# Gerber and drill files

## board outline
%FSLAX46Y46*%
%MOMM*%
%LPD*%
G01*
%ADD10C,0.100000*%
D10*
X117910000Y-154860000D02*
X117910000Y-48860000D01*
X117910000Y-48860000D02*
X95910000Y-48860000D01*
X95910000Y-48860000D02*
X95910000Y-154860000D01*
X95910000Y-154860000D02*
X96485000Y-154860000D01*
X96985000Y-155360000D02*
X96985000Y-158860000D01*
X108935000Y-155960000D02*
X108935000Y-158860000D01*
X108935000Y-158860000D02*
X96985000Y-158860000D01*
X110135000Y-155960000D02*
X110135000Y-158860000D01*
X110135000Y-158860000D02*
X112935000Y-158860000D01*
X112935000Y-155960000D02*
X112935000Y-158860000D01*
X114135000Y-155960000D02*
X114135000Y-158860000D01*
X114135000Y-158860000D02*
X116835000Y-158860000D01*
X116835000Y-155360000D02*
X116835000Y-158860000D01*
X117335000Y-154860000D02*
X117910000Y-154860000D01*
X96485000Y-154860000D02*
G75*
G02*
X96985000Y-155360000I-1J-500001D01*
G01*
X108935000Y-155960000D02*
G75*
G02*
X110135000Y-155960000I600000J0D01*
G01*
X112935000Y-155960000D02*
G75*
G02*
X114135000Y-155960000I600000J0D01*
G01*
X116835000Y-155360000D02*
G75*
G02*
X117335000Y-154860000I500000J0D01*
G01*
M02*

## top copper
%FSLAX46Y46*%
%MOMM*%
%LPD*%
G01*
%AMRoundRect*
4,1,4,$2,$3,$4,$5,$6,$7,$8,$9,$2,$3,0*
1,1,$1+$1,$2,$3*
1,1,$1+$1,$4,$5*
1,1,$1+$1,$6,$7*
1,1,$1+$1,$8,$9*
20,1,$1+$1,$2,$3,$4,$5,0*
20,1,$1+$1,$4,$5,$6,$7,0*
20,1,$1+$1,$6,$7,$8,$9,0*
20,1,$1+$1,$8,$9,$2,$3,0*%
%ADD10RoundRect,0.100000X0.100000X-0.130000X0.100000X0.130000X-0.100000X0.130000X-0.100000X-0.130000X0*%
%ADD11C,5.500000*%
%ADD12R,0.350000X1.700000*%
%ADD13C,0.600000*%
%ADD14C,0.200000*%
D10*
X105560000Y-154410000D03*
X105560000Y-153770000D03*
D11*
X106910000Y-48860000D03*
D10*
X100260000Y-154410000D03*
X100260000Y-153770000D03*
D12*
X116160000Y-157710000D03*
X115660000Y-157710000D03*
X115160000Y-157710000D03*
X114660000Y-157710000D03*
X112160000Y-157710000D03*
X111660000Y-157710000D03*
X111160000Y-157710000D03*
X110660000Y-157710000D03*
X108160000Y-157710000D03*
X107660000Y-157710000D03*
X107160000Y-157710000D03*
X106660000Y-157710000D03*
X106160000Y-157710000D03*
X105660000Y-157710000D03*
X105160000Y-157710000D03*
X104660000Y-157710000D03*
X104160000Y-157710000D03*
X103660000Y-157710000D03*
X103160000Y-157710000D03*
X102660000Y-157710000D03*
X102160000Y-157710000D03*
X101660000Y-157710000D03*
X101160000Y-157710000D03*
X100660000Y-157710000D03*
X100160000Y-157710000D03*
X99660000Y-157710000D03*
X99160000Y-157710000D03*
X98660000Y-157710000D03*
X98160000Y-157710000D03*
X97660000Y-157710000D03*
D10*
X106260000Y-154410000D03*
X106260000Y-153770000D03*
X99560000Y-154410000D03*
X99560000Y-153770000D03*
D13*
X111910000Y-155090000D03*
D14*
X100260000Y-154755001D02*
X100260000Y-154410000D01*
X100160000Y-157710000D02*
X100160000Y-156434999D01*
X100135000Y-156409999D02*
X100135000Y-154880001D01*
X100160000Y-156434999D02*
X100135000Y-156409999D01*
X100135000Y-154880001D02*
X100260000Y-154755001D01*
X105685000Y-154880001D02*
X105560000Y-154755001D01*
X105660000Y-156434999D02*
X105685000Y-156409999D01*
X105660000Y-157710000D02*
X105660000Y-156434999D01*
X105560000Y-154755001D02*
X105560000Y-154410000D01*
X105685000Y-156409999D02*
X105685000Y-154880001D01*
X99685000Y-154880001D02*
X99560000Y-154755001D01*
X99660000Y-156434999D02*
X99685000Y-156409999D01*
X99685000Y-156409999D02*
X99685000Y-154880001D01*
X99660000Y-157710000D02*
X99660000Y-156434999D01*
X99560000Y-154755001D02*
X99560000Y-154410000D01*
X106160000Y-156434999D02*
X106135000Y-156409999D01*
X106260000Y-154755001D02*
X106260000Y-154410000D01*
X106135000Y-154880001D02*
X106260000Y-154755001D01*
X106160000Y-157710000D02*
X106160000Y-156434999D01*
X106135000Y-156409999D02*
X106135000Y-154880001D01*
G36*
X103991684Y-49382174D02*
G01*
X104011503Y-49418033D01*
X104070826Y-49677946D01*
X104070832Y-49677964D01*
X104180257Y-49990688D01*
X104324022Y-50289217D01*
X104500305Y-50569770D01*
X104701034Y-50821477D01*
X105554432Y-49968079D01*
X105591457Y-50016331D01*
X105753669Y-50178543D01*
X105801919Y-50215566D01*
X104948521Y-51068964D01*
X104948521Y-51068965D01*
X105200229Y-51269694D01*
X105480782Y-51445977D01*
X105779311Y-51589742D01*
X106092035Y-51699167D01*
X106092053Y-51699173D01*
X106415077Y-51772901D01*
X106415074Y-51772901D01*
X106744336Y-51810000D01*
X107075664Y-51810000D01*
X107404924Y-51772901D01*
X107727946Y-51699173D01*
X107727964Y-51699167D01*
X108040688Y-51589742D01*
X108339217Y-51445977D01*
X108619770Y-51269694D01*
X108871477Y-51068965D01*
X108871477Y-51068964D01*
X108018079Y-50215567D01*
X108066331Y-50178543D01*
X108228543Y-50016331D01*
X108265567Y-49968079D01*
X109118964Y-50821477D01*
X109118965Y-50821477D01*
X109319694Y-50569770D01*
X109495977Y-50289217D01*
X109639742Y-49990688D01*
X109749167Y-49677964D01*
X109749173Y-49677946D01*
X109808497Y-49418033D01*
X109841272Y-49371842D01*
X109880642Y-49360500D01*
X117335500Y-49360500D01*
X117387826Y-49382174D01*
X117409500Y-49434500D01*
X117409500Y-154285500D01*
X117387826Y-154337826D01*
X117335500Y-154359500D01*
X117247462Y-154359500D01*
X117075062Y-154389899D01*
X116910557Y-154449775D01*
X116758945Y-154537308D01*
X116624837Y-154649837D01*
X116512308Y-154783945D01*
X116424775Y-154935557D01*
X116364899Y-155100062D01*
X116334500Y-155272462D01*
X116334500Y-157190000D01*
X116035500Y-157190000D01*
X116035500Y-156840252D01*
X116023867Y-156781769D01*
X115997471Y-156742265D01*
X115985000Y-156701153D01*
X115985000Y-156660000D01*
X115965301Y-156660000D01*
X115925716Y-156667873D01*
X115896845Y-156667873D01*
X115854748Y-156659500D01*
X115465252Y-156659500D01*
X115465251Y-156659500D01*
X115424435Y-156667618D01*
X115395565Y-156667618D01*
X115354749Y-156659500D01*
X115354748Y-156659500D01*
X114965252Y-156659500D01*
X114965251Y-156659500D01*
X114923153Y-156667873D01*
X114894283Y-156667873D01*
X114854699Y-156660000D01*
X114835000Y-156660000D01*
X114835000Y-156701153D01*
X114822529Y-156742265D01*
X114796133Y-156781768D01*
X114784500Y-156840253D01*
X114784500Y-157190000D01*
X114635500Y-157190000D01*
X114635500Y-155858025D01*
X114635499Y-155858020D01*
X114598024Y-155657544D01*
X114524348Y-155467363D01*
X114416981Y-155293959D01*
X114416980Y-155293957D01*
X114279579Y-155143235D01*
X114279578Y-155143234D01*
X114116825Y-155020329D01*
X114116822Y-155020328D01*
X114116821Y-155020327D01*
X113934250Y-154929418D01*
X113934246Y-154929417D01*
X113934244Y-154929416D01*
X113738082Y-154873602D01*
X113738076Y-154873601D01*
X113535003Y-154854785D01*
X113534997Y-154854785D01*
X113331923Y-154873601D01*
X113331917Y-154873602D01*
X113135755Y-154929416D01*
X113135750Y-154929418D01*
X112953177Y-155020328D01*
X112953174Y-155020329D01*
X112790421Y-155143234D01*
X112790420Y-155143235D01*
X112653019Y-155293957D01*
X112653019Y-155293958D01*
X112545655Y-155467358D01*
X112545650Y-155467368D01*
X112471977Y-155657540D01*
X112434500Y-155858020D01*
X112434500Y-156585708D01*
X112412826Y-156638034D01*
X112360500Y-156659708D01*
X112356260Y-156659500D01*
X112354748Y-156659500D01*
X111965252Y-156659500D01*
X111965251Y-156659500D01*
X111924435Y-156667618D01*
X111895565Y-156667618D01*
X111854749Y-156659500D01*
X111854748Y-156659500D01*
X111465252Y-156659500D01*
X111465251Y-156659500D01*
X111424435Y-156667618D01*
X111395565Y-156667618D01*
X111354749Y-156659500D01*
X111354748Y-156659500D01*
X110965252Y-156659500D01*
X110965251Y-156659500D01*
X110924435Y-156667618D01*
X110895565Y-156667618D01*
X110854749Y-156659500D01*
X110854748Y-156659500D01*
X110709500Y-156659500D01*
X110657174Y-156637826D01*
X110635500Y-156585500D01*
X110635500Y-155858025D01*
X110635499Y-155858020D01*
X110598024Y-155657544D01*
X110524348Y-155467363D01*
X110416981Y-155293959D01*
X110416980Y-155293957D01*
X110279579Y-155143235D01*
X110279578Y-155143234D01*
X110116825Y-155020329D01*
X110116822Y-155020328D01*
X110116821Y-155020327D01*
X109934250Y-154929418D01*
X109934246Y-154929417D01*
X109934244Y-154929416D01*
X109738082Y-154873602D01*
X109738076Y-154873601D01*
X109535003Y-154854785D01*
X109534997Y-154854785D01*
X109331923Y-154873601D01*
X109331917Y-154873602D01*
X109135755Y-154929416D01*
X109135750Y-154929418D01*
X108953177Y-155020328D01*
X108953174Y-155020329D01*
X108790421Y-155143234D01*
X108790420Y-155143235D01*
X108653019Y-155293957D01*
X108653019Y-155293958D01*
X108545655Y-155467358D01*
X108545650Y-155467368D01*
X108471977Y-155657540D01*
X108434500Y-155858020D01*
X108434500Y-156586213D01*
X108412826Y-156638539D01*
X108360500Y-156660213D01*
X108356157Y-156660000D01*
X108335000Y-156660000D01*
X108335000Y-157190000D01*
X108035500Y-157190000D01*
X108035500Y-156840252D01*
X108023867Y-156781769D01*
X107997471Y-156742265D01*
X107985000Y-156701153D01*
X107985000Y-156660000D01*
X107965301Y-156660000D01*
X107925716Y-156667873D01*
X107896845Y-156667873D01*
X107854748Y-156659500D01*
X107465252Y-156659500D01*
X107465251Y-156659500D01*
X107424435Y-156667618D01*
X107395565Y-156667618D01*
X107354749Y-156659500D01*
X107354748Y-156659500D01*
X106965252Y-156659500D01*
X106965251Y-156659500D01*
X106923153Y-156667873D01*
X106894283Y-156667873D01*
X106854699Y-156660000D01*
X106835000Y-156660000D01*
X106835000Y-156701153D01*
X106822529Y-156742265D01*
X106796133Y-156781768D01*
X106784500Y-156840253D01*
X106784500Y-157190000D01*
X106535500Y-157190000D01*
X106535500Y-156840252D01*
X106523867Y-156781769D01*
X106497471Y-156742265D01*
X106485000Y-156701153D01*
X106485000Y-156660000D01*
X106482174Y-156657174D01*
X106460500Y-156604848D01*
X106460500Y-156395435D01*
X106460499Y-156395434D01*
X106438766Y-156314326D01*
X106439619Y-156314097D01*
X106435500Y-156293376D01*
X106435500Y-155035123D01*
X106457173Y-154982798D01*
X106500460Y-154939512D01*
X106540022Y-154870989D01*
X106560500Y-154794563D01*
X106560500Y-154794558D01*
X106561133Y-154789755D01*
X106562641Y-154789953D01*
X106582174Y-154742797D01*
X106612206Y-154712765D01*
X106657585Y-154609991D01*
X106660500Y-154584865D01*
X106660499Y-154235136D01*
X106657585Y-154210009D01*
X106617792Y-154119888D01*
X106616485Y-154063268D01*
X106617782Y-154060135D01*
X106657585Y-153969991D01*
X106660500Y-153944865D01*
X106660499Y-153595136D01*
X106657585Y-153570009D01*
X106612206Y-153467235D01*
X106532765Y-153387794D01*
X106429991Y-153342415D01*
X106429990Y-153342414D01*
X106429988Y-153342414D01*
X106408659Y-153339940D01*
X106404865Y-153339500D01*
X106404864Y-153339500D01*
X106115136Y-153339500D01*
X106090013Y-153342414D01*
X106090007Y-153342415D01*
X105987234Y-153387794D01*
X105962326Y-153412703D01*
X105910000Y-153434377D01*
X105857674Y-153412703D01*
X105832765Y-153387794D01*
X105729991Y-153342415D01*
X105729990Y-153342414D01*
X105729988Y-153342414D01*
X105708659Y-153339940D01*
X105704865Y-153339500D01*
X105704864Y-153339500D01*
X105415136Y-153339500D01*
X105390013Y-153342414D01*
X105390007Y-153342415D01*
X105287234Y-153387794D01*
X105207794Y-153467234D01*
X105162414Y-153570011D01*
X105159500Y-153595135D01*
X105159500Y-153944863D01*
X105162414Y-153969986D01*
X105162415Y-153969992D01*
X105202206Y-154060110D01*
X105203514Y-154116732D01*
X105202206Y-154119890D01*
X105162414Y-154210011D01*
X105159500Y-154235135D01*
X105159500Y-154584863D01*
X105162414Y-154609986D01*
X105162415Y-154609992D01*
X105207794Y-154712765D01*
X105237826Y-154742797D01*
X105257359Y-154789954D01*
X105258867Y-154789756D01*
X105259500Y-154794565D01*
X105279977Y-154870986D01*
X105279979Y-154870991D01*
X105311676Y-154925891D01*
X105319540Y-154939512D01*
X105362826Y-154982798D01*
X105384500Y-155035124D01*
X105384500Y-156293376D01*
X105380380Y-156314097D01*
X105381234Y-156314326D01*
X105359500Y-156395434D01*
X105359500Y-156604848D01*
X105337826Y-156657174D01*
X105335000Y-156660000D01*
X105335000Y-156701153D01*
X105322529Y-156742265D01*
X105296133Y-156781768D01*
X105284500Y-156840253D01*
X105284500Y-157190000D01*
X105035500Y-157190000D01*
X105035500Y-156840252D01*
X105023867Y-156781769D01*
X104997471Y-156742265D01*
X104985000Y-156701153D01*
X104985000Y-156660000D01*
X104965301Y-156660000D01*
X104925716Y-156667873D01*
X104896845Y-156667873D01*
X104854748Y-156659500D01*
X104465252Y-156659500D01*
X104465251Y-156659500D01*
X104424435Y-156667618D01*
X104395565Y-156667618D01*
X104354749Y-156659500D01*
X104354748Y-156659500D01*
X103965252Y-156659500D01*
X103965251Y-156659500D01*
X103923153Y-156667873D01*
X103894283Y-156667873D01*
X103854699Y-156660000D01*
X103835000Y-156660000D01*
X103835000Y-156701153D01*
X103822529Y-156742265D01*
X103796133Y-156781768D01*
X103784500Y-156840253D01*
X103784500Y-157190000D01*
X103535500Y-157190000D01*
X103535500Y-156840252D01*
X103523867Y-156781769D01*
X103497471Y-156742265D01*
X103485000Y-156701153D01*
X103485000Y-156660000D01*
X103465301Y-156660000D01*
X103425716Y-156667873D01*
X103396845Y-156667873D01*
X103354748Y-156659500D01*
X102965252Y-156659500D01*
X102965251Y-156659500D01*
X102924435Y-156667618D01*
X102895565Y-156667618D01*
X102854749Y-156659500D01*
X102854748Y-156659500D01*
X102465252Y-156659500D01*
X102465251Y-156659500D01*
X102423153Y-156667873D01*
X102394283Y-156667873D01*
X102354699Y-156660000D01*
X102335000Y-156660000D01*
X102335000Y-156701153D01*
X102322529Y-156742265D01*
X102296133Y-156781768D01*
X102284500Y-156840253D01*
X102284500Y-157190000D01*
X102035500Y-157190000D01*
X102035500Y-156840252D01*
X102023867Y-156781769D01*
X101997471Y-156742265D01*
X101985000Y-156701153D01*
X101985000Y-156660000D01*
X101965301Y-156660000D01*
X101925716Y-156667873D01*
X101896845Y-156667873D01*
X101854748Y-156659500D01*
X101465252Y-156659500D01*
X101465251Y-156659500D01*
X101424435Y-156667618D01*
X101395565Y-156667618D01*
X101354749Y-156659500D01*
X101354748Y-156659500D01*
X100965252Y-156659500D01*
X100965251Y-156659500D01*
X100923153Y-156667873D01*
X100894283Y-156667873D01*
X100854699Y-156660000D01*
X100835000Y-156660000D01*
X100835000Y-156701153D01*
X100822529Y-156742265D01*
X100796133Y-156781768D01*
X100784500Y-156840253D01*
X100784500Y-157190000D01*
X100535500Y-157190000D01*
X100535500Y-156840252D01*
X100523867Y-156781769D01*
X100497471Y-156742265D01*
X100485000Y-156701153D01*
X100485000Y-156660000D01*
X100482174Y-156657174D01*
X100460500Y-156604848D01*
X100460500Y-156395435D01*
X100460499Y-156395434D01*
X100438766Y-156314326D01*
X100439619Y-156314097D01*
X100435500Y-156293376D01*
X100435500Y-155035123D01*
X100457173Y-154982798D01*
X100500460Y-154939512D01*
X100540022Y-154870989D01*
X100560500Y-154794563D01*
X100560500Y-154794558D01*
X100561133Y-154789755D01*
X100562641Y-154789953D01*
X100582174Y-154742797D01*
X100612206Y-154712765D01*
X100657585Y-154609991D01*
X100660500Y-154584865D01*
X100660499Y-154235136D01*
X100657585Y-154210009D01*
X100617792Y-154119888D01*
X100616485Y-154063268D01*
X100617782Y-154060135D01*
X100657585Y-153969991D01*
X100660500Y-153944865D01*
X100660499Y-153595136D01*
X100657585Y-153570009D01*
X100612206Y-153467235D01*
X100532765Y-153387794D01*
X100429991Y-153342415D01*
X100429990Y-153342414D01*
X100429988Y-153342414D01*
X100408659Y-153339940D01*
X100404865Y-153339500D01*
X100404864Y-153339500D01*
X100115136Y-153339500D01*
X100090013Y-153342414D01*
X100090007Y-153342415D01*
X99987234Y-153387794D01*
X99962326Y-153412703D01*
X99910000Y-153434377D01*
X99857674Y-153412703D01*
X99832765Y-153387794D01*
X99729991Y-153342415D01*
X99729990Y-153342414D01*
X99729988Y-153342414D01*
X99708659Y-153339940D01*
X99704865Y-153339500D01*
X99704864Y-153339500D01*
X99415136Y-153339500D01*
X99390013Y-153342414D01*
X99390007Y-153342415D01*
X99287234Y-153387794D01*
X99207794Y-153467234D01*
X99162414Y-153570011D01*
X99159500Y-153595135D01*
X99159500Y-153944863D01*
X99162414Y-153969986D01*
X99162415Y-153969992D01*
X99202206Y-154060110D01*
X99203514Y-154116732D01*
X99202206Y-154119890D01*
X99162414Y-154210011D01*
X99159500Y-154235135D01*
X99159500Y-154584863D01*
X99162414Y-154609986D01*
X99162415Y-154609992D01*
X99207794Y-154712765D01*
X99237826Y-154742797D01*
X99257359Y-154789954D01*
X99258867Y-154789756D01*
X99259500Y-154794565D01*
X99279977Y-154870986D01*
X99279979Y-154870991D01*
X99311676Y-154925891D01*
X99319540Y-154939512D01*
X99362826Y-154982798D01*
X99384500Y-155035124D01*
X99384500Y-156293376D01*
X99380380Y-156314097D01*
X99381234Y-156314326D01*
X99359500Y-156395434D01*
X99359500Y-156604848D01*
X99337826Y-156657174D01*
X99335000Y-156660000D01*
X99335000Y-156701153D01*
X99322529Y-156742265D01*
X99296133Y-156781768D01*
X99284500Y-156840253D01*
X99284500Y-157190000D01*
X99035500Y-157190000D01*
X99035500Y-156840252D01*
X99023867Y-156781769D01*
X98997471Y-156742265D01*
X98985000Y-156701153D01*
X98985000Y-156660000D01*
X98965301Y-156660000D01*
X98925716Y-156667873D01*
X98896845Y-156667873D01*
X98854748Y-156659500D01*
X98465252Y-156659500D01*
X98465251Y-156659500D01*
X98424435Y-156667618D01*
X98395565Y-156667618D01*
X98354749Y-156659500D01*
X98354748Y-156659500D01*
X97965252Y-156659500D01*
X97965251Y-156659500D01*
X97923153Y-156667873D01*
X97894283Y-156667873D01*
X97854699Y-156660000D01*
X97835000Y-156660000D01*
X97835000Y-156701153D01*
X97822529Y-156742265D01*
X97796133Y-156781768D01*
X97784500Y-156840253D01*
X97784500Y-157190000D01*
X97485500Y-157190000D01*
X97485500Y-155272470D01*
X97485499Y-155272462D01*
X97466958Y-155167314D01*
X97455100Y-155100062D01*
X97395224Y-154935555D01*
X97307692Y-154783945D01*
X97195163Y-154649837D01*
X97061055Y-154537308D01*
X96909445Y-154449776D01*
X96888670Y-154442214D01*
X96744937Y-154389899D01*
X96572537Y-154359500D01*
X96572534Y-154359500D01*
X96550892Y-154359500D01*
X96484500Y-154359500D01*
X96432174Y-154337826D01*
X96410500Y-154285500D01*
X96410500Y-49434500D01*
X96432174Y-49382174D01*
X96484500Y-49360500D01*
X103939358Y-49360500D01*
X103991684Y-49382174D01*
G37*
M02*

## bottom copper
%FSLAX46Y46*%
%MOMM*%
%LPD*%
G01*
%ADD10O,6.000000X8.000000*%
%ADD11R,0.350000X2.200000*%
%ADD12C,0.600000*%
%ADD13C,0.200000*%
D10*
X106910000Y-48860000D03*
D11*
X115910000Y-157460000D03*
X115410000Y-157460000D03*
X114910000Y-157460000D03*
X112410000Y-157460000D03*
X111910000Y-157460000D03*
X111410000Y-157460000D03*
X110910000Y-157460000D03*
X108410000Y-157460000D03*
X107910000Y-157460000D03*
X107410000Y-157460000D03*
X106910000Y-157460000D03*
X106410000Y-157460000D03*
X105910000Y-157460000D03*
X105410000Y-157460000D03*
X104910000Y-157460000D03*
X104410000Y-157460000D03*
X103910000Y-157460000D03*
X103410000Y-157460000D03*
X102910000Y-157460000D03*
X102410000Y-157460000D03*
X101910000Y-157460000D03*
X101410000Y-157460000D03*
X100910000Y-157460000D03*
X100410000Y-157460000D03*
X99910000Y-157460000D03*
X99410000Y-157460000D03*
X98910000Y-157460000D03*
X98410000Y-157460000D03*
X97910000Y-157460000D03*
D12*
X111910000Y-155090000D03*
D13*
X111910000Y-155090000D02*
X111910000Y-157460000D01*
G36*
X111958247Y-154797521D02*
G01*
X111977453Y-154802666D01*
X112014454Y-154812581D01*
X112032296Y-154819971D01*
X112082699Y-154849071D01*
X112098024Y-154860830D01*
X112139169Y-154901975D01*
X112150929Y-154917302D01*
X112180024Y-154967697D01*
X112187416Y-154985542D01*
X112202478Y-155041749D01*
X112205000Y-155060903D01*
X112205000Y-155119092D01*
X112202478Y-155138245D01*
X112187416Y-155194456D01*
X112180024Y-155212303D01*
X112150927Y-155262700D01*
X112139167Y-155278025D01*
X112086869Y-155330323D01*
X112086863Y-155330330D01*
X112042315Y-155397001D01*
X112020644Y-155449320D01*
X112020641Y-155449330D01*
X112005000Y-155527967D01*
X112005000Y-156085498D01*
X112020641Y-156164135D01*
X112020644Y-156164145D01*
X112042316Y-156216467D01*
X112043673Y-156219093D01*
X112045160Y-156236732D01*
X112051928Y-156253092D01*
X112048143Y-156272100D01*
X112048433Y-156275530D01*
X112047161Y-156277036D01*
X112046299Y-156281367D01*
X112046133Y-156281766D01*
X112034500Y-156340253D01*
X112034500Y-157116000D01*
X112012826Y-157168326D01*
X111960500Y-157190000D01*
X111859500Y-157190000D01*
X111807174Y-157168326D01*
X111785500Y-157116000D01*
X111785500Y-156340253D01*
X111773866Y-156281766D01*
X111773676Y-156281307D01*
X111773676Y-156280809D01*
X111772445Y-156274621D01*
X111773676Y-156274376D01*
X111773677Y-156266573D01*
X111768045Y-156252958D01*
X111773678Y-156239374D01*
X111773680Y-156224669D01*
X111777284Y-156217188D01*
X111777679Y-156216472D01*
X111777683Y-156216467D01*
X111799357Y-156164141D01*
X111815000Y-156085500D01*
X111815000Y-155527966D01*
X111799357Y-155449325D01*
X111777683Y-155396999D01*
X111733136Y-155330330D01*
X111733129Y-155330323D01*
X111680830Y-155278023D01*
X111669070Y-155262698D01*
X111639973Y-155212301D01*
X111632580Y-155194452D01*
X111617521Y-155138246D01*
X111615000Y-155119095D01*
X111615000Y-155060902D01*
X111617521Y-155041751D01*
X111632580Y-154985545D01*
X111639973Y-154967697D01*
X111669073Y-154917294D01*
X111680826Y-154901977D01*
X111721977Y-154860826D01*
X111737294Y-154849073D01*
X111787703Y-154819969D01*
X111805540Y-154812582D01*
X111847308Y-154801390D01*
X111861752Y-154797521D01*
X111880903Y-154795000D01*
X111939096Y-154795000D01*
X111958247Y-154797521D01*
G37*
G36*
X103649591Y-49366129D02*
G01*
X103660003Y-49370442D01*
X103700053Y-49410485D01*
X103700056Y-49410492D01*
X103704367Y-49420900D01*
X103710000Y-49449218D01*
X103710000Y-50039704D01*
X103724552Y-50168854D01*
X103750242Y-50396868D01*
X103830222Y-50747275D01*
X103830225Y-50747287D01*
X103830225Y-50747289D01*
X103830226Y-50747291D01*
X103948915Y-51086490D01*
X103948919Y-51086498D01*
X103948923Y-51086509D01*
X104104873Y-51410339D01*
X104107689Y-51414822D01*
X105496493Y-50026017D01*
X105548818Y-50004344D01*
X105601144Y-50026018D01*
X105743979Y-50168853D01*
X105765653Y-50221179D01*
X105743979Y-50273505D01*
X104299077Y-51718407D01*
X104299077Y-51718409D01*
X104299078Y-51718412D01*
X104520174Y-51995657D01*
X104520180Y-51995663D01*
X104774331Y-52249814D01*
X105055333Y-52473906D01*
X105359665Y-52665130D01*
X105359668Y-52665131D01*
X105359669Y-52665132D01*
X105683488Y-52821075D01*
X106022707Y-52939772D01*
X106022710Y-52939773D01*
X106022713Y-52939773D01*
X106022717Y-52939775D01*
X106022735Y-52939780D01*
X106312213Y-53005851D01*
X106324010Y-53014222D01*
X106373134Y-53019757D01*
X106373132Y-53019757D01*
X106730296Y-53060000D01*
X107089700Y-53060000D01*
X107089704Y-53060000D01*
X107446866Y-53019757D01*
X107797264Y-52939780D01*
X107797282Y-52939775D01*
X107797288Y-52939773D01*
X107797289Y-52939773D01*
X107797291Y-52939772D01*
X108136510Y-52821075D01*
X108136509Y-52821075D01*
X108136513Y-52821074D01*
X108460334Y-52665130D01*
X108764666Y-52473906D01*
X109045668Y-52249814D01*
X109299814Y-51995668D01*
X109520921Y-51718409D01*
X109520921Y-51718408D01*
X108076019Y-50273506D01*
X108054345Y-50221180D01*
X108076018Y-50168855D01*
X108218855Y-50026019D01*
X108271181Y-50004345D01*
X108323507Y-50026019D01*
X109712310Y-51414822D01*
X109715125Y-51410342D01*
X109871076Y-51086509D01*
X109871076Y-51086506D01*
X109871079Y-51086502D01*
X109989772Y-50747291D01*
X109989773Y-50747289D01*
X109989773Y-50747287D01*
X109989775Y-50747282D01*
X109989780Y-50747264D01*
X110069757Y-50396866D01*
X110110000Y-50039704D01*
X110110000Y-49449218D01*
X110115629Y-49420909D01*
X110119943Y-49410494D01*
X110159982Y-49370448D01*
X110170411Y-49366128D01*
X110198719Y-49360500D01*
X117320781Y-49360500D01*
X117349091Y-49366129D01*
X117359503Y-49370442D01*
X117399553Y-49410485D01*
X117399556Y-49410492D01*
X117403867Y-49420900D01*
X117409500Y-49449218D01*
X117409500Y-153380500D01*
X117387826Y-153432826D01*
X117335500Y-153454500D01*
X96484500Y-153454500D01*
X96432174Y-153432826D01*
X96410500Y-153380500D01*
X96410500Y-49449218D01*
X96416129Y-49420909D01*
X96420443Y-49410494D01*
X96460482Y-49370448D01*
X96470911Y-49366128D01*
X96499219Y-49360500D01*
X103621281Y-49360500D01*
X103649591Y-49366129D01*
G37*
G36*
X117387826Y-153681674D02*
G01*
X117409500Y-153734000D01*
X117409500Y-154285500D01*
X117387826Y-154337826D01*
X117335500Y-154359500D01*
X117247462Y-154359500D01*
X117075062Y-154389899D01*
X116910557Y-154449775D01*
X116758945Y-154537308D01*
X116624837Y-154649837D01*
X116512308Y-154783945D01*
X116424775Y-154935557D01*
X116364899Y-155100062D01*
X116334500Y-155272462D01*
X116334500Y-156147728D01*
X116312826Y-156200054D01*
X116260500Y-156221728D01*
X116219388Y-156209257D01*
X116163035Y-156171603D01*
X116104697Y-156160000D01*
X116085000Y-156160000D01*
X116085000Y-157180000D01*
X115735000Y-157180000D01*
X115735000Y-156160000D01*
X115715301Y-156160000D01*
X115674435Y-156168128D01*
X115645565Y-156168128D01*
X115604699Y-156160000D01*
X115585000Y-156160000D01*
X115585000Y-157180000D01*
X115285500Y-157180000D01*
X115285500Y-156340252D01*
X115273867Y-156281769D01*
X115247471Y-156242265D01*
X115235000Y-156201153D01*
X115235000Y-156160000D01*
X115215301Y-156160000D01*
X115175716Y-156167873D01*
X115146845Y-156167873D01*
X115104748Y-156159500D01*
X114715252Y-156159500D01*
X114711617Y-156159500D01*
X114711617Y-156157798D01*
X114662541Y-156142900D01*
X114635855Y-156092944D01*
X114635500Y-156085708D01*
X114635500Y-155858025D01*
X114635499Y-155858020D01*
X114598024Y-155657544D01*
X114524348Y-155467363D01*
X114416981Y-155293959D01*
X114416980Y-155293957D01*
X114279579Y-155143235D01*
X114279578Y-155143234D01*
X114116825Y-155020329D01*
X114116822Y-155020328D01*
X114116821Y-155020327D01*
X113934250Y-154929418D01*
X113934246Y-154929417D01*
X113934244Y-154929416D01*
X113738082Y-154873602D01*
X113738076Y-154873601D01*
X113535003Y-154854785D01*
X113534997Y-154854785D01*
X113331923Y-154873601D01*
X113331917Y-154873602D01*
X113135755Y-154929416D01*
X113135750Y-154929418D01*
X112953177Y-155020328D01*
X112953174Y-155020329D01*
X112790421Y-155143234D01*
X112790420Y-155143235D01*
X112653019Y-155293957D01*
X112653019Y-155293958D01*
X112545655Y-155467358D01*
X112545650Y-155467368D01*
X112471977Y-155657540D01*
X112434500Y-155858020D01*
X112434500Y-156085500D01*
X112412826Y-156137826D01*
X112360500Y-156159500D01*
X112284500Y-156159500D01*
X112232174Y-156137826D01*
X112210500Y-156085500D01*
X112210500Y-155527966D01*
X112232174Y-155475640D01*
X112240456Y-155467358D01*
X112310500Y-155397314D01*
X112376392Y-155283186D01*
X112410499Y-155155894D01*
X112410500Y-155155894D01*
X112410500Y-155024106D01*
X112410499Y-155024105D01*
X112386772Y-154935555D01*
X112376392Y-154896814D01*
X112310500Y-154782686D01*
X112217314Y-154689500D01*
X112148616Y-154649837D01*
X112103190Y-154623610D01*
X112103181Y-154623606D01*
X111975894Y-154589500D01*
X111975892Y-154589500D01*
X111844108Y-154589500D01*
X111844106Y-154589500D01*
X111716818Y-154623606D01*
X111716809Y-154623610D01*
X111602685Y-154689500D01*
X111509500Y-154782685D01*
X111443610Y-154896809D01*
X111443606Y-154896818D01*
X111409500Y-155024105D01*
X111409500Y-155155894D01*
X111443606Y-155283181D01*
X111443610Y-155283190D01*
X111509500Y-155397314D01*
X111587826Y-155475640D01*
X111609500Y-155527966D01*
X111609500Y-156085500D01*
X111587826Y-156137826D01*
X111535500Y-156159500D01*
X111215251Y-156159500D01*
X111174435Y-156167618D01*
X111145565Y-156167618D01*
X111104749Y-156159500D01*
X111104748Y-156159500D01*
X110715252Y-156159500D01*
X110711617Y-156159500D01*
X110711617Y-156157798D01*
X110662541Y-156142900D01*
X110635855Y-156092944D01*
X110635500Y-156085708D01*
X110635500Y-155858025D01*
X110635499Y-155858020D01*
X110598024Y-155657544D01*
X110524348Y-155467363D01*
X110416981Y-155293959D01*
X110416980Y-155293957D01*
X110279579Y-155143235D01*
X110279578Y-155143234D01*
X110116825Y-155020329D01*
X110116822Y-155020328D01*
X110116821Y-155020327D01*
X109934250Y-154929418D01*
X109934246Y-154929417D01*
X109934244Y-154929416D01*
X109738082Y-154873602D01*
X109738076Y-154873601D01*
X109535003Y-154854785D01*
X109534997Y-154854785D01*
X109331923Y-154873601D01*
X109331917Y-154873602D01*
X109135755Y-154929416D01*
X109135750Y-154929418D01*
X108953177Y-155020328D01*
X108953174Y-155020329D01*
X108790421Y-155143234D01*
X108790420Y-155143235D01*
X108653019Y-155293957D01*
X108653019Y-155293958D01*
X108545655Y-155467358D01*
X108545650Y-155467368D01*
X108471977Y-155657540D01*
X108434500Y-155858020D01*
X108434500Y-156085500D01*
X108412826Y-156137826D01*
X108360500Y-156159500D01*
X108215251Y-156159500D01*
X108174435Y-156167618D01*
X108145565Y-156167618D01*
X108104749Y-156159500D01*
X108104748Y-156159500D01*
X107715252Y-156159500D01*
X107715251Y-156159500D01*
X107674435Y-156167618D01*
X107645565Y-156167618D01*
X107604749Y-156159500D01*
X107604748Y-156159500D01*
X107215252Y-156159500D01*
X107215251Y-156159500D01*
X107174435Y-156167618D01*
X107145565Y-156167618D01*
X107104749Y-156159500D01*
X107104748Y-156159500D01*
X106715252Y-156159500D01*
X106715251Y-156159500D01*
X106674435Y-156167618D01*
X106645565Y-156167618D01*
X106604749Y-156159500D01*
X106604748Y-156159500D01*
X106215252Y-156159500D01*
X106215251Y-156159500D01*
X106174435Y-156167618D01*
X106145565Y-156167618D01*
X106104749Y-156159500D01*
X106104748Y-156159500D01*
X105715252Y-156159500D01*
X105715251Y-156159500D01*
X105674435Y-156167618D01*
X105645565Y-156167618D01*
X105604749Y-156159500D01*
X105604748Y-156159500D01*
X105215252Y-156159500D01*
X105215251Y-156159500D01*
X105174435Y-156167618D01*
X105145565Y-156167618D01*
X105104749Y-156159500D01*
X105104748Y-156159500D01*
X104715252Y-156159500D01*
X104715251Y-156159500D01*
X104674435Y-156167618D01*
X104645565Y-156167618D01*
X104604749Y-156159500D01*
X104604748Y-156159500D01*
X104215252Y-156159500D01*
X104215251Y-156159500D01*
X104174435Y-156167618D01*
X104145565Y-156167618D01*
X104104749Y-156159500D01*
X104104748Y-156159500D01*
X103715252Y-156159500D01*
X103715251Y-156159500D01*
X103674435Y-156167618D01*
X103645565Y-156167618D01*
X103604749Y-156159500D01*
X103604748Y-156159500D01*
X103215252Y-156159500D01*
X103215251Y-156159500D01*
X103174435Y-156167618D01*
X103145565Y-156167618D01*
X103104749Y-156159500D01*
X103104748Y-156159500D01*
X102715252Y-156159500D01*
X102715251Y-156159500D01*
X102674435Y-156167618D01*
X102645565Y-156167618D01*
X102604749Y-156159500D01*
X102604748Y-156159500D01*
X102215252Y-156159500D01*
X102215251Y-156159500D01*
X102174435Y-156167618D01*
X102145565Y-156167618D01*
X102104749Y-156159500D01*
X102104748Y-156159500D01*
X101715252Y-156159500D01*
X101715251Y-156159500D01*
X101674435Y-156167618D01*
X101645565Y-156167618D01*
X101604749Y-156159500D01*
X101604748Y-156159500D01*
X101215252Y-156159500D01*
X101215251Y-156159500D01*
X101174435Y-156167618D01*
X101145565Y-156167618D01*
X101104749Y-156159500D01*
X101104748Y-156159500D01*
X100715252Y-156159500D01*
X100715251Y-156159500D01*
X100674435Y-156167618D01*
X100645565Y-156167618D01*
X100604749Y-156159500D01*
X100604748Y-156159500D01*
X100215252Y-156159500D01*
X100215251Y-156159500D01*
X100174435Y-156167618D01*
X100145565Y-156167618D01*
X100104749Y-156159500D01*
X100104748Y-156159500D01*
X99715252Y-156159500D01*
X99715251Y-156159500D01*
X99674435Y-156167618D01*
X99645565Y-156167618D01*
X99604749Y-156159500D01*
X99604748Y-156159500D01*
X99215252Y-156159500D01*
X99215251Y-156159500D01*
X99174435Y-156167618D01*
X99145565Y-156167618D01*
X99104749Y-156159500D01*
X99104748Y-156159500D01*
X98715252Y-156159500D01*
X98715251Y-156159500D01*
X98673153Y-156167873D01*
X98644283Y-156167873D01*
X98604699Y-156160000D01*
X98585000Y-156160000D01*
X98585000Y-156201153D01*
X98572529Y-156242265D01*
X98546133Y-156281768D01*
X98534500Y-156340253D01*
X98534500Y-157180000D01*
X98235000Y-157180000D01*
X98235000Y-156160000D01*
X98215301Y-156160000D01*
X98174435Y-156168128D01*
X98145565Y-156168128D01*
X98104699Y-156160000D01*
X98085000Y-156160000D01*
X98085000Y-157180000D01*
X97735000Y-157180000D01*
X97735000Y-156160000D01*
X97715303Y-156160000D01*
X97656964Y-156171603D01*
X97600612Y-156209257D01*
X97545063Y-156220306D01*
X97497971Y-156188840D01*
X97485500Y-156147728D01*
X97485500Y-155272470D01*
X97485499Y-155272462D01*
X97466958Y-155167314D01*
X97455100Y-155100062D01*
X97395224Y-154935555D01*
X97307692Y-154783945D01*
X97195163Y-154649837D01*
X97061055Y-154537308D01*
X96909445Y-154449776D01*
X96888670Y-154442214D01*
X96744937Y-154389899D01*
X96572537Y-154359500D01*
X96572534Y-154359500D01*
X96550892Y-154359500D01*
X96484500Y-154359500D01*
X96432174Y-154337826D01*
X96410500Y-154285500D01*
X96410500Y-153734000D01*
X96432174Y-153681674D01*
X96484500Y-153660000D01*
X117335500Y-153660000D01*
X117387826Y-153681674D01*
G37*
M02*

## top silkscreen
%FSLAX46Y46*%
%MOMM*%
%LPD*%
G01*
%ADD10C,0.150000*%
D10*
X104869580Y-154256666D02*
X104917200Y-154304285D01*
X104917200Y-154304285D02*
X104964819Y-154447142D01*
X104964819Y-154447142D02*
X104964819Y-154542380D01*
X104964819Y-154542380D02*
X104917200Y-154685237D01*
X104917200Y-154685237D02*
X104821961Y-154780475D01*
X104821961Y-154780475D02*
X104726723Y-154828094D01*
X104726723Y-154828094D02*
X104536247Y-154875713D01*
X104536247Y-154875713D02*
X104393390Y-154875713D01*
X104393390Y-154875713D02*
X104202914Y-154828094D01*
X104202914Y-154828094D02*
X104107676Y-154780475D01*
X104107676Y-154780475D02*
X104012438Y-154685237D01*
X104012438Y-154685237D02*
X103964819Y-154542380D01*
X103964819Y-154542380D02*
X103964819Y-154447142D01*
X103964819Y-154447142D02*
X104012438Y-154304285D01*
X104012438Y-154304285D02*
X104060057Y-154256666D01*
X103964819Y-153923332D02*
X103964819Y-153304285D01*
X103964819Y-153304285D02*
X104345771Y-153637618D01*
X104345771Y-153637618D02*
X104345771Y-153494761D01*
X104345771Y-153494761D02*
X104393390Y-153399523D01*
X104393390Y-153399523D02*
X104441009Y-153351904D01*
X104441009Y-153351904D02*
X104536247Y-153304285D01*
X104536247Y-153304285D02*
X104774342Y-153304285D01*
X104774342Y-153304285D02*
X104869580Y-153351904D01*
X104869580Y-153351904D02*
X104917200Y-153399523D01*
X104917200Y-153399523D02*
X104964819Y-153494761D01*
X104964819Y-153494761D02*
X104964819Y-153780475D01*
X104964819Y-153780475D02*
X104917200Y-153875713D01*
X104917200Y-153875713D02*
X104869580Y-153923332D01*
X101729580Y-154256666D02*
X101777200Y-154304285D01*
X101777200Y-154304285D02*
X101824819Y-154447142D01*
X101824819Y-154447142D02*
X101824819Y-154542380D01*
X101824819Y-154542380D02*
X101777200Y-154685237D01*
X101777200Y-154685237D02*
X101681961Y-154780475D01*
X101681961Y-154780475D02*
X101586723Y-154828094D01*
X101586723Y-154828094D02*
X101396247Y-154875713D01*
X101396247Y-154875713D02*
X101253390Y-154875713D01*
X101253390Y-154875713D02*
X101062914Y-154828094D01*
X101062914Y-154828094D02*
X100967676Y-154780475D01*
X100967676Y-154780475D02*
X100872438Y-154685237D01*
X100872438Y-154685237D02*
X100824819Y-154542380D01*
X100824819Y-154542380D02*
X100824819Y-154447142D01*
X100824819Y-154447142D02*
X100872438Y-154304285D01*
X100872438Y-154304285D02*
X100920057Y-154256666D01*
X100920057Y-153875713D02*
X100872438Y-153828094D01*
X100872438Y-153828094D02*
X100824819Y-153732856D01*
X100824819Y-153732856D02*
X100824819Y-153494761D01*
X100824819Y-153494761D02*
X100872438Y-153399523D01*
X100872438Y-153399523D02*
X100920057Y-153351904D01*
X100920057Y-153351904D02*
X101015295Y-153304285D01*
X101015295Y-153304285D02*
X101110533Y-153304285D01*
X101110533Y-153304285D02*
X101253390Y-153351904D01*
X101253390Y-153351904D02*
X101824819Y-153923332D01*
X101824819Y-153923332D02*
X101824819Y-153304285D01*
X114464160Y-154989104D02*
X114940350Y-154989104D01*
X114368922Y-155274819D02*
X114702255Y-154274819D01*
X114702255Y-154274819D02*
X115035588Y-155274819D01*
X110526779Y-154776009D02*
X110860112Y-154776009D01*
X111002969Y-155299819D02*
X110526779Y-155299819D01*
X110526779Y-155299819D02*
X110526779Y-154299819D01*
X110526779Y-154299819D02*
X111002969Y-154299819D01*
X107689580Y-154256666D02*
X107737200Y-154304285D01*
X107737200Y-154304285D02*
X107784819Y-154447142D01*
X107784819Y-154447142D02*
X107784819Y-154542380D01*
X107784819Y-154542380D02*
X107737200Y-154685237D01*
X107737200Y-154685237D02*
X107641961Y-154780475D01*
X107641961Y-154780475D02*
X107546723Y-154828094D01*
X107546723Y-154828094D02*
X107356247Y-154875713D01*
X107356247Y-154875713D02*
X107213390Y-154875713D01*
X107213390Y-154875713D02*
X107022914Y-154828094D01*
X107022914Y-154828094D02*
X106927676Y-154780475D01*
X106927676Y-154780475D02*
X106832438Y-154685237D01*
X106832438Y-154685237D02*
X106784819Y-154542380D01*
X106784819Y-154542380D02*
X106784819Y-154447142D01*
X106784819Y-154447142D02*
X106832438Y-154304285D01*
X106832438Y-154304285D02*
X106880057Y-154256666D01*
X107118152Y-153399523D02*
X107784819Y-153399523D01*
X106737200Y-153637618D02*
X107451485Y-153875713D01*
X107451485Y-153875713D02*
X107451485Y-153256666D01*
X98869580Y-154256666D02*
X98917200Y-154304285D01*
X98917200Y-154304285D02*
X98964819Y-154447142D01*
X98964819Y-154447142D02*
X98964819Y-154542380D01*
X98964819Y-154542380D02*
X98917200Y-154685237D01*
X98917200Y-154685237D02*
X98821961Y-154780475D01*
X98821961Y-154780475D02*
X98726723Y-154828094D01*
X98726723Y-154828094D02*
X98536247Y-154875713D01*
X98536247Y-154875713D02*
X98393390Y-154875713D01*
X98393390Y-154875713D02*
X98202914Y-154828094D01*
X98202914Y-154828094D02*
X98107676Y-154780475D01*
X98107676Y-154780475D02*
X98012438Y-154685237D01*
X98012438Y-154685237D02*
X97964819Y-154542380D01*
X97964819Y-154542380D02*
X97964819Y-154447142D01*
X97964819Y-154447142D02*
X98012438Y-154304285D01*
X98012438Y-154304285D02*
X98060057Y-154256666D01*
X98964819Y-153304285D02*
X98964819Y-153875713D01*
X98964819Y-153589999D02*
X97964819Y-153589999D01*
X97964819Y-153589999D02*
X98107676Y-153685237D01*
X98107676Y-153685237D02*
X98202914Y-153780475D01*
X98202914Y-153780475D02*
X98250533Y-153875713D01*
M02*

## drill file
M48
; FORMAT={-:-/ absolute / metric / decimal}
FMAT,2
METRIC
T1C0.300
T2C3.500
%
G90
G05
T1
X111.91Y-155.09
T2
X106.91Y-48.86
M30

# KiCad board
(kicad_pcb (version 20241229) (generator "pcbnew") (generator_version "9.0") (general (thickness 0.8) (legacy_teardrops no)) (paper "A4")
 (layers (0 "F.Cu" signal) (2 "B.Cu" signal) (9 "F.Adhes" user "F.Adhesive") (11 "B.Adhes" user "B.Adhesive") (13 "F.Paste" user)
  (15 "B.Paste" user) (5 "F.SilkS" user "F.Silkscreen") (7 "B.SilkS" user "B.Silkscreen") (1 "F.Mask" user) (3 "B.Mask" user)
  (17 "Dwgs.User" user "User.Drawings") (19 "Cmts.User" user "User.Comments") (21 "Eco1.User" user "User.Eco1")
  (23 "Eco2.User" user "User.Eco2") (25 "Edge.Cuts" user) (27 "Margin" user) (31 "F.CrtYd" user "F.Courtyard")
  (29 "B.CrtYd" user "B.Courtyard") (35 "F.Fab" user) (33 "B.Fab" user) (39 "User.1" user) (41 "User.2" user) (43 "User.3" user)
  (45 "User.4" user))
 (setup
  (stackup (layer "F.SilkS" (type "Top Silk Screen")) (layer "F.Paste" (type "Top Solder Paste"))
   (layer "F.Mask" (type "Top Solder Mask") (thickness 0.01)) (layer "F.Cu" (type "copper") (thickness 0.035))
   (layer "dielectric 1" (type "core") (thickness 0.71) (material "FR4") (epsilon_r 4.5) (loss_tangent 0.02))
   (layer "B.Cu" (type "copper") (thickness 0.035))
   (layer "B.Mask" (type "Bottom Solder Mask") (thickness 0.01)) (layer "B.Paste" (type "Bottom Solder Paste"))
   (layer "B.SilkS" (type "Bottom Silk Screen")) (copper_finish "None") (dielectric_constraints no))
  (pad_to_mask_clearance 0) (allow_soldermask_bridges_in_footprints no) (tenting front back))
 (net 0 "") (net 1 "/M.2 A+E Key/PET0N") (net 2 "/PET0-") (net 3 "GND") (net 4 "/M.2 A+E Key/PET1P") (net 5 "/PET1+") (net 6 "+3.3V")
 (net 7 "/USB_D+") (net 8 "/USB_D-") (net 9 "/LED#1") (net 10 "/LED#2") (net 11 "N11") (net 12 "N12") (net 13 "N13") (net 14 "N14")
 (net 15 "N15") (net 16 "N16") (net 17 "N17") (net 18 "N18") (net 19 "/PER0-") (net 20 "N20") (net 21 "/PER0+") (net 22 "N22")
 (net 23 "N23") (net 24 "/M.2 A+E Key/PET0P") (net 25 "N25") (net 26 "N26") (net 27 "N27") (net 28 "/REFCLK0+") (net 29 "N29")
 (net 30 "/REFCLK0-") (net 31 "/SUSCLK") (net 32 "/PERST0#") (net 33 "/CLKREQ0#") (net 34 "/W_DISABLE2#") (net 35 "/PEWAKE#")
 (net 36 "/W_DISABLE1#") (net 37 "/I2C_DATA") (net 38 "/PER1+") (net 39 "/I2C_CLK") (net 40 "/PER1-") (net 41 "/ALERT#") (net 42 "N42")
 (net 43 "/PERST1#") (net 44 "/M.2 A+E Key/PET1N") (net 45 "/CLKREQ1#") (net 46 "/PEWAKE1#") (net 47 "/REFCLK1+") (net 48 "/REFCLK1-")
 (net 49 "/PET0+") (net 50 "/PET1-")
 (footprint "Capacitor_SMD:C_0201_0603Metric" (layer "F.Cu") (at 105.56 154.09 90)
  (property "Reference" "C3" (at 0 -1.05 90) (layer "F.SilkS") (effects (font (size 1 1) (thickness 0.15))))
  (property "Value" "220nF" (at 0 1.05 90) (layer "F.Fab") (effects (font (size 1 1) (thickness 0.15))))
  (pad "" smd roundrect (at -0.345 0 90) (size 0.318 0.36) (layers "F.Paste") (roundrect_rratio 0.25))
  (pad "" smd roundrect (at 0.345 0 90) (size 0.318 0.36) (layers "F.Paste") (roundrect_rratio 0.25))
  (pad "1" smd roundrect (at -0.32 0 90) (size 0.46 0.4) (layers "F.Cu" "F.Mask") (roundrect_rratio 0.25) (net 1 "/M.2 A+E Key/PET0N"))
  (pad "2" smd roundrect (at 0.32 0 90) (size 0.46 0.4) (layers "F.Cu" "F.Mask") (roundrect_rratio 0.25) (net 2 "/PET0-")))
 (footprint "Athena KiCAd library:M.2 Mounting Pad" (layer "F.Cu") (at 106.91 48.86)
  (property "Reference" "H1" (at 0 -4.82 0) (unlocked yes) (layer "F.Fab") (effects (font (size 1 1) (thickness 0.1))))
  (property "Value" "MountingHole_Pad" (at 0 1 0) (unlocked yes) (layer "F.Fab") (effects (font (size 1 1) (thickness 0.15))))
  (pad "1" thru_hole circle (at 0 0) (size 5.5 5.5) (drill 3.5) (layers "*.Cu" "*.Mask") (remove_unused_layers no) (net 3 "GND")
   (padstack (mode front_inner_back)
    (layer "Inner" (shape circle) (size 5.5 5.5) (zone_connect -1))
    (layer "B.Cu" (shape oval) (size 6 8) (thermal_bridge_angle 45) (zone_connect -1)))))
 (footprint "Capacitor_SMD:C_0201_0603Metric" (layer "F.Cu") (at 100.26 154.09 90)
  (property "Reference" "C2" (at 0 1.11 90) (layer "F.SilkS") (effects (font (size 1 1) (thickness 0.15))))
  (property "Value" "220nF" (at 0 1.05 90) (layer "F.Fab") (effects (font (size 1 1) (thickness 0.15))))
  (pad "" smd roundrect (at -0.345 0 90) (size 0.318 0.36) (layers "F.Paste") (roundrect_rratio 0.25))
  (pad "" smd roundrect (at 0.345 0 90) (size 0.318 0.36) (layers "F.Paste") (roundrect_rratio 0.25))
  (pad "1" smd roundrect (at -0.32 0 90) (size 0.46 0.4) (layers "F.Cu" "F.Mask") (roundrect_rratio 0.25) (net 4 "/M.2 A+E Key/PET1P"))
  (pad "2" smd roundrect (at 0.32 0 90) (size 0.46 0.4) (layers "F.Cu" "F.Mask") (roundrect_rratio 0.25) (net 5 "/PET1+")))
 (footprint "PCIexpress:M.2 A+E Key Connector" (layer "F.Cu") (at 106.91 157.75)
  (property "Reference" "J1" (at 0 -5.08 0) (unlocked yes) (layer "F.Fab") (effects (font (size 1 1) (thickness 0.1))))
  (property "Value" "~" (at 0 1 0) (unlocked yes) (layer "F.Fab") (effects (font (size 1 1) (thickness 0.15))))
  (fp_line (start -11 -2.89) (end -10.425 -2.89) (stroke (width 0.1) (type default)) (layer "Edge.Cuts"))
  (fp_line (start -9.925 -2.39) (end -9.925 1.11) (stroke (width 0.1) (type default)) (layer "Edge.Cuts"))
  (fp_line (start 2.025 -1.79) (end 2.025 1.11) (stroke (width 0.1) (type default)) (layer "Edge.Cuts"))
  (fp_line (start 2.025 1.11) (end -9.925 1.11) (stroke (width 0.1) (type default)) (layer "Edge.Cuts"))
  (fp_line (start 3.225 -1.79) (end 3.225 1.11) (stroke (width 0.1) (type default)) (layer "Edge.Cuts"))
  (fp_line (start 3.225 1.11) (end 6.025 1.11) (stroke (width 0.1) (type default)) (layer "Edge.Cuts"))
  (fp_line (start 6.025 -1.79) (end 6.025 1.11) (stroke (width 0.1) (type default)) (layer "Edge.Cuts"))
  (fp_line (start 7.225 -1.79) (end 7.225 1.11) (stroke (width 0.1) (type default)) (layer "Edge.Cuts"))
  (fp_line (start 7.225 1.11) (end 9.925 1.11) (stroke (width 0.1) (type default)) (layer "Edge.Cuts"))
  (fp_line (start 9.925 -2.39) (end 9.925 1.11) (stroke (width 0.1) (type default)) (layer "Edge.Cuts"))
  (fp_line (start 10.425 -2.89) (end 11 -2.89) (stroke (width 0.1) (type default)) (layer "Edge.Cuts"))
  (fp_arc (start -10.425 -2.89) (mid -10.071447 -2.743553) (end -9.925 -2.39) (stroke (width 0.1) (type default)) (layer "Edge.Cuts"))
  (fp_arc (start 2.025 -1.79) (mid 2.625 -2.39) (end 3.225 -1.79) (stroke (width 0.1) (type default)) (layer "Edge.Cuts"))
  (fp_arc (start 6.025 -1.79) (mid 6.625 -2.39) (end 7.225 -1.79) (stroke (width 0.1) (type default)) (layer "Edge.Cuts"))
  (fp_arc (start 9.925 -2.39) (mid 10.071447 -2.743553) (end 10.425 -2.89) (stroke (width 0.1) (type default)) (layer "Edge.Cuts"))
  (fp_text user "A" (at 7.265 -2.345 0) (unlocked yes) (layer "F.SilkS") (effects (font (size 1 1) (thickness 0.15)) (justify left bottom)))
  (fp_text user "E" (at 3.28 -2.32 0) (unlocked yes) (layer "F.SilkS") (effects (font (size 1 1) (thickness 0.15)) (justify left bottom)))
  (pad "1" smd rect (at 9.25 -0.04 180) (size 0.35 1.7) (layers "F.Cu") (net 3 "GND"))
  (pad "2" smd rect (at 9 -0.29 180) (size 0.35 2.2) (layers "B.Cu") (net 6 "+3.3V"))
  (pad "3" smd rect (at 8.75 -0.04 180) (size 0.35 1.7) (layers "F.Cu") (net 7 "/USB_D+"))
  (pad "4" smd rect (at 8.5 -0.29 180) (size 0.35 2.2) (layers "B.Cu") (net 6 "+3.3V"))
  (pad "5" smd rect (at 8.25 -0.04 180) (size 0.35 1.7) (layers "F.Cu") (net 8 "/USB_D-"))
  (pad "6" smd rect (at 8 -0.29 180) (size 0.35 2.2) (layers "B.Cu") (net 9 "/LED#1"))
  (pad "7" smd rect (at 7.75 -0.04 180) (size 0.35 1.7) (layers "F.Cu") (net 3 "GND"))
  (pad "16" smd rect (at 5.5 -0.29 180) (size 0.35 2.2) (layers "B.Cu") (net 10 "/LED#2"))
  (pad "17" smd rect (at 5.25 -0.04 180) (size 0.35 1.7) (layers "F.Cu") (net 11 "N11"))
  (pad "18" smd rect (at 5 -0.29 180) (size 0.35 2.2) (layers "B.Cu") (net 3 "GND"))
  (pad "19" smd rect (at 4.75 -0.04 180) (size 0.35 1.7) (layers "F.Cu") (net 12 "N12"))
  (pad "20" smd rect (at 4.5 -0.29 180) (size 0.35 2.2) (layers "B.Cu") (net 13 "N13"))
  (pad "21" smd rect (at 4.25 -0.04 180) (size 0.35 1.7) (layers "F.Cu") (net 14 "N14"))
  (pad "22" smd rect (at 4 -0.29 180) (size 0.35 2.2) (layers "B.Cu") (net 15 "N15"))
  (pad "23" smd rect (at 3.75 -0.04 180) (size 0.35 1.7) (layers "F.Cu") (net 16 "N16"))
  (pad "32" smd rect (at 1.5 -0.29 180) (size 0.35 2.2) (layers "B.Cu") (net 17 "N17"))
  (pad "33" smd rect (at 1.25 -0.04 180) (size 0.35 1.7) (layers "F.Cu") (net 3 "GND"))
  (pad "34" smd rect (at 1 -0.29 180) (size 0.35 2.2) (layers "B.Cu") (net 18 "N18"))
  (pad "35" smd rect (at 0.75 -0.04 180) (size 0.35 1.7) (layers "F.Cu") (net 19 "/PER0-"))
  (pad "36" smd rect (at 0.5 -0.29 180) (size 0.35 2.2) (layers "B.Cu") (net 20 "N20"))
  (pad "37" smd rect (at 0.25 -0.04 180) (size 0.35 1.7) (layers "F.Cu") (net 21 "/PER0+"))
  (pad "38" smd rect (at 0 -0.29 180) (size 0.35 2.2) (layers "B.Cu") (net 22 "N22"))
  (pad "39" smd rect (at -0.25 -0.04 180) (size 0.35 1.7) (layers "F.Cu") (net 3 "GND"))
  (pad "40" smd rect (at -0.5 -0.29 180) (size 0.35 2.2) (layers "B.Cu") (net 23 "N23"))
  (pad "41" smd rect (at -0.75 -0.04 180) (size 0.35 1.7) (layers "F.Cu") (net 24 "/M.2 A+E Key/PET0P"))
  (pad "42" smd rect (at -1 -0.29 180) (size 0.35 2.2) (layers "B.Cu") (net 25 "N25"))
  (pad "43" smd rect (at -1.25 -0.04 180) (size 0.35 1.7) (layers "F.Cu") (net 1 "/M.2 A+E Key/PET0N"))
  (pad "44" smd rect (at -1.5 -0.29 180) (size 0.35 2.2) (layers "B.Cu") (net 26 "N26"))
  (pad "45" smd rect (at -1.75 -0.04 180) (size 0.35 1.7) (layers "F.Cu") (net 3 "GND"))
  (pad "46" smd rect (at -2 -0.29 180) (size 0.35 2.2) (layers "B.Cu") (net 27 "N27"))
  (pad "47" smd rect (at -2.25 -0.04 180) (size 0.35 1.7) (layers "F.Cu") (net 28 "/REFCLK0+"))
  (pad "48" smd rect (at -2.5 -0.29 180) (size 0.35 2.2) (layers "B.Cu") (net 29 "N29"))
  (pad "49" smd rect (at -2.75 -0.04 180) (size 0.35 1.7) (layers "F.Cu") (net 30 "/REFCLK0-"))
  (pad "50" smd rect (at -3 -0.29 180) (size 0.35 2.2) (layers "B.Cu") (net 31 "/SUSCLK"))
  (pad "51" smd rect (at -3.25 -0.04 180) (size 0.35 1.7) (layers "F.Cu") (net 3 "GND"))
  (pad "52" smd rect (at -3.5 -0.29 180) (size 0.35 2.2) (layers "B.Cu") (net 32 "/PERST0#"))
  (pad "53" smd rect (at -3.75 -0.04 180) (size 0.35 1.7) (layers "F.Cu") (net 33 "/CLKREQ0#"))
  (pad "54" smd rect (at -4 -0.29 180) (size 0.35 2.2) (layers "B.Cu") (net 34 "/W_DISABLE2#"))
  (pad "55" smd rect (at -4.25 -0.04 180) (size 0.35 1.7) (layers "F.Cu") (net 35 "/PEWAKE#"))
  (pad "56" smd rect (at -4.5 -0.29 180) (size 0.35 2.2) (layers "B.Cu") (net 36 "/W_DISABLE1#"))
  (pad "57" smd rect (at -4.75 -0.04 180) (size 0.35 1.7) (layers "F.Cu") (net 3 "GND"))
  (pad "58" smd rect (at -5 -0.29 180) (size 0.35 2.2) (layers "B.Cu") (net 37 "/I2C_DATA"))
  (pad "59" smd rect (at -5.25 -0.04 180) (size 0.35 1.7) (layers "F.Cu") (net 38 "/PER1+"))
  (pad "60" smd rect (at -5.5 -0.29 180) (size 0.35 2.2) (layers "B.Cu") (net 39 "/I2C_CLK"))
  (pad "61" smd rect (at -5.75 -0.04 180) (size 0.35 1.7) (layers "F.Cu") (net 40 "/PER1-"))
  (pad "62" smd rect (at -6 -0.29 180) (size 0.35 2.2) (layers "B.Cu") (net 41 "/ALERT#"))
  (pad "63" smd rect (at -6.25 -0.04 180) (size 0.35 1.7) (layers "F.Cu") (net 3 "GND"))
  (pad "64" smd rect (at -6.5 -0.29 180) (size 0.35 2.2) (layers "B.Cu") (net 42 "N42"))
  (pad "65" smd rect (at -6.75 -0.04 180) (size 0.35 1.7) (layers "F.Cu") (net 4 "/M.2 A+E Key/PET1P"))
  (pad "66" smd rect (at -7 -0.29 180) (size 0.35 2.2) (layers "B.Cu") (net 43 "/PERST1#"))
  (pad "67" smd rect (at -7.25 -0.04 180) (size 0.35 1.7) (layers "F.Cu") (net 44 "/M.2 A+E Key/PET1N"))
  (pad "68" smd rect (at -7.5 -0.29 180) (size 0.35 2.2) (layers "B.Cu") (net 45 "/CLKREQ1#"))
  (pad "69" smd rect (at -7.75 -0.04 180) (size 0.35 1.7) (layers "F.Cu") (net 3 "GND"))
  (pad "70" smd rect (at -8 -0.29 180) (size 0.35 2.2) (layers "B.Cu") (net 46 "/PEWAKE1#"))
  (pad "71" smd rect (at -8.25 -0.04 180) (size 0.35 1.7) (layers "F.Cu") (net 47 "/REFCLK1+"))
  (pad "72" smd rect (at -8.5 -0.29 180) (size 0.35 2.2) (layers "B.Cu") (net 6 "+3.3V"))
  (pad "73" smd rect (at -8.75 -0.04 180) (size 0.35 1.7) (layers "F.Cu") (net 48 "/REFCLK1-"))
  (pad "74" smd rect (at -9 -0.29 180) (size 0.35 2.2) (layers "B.Cu") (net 6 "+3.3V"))
  (pad "75" smd rect (at -9.25 -0.04 180) (size 0.35 1.7) (layers "F.Cu") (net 3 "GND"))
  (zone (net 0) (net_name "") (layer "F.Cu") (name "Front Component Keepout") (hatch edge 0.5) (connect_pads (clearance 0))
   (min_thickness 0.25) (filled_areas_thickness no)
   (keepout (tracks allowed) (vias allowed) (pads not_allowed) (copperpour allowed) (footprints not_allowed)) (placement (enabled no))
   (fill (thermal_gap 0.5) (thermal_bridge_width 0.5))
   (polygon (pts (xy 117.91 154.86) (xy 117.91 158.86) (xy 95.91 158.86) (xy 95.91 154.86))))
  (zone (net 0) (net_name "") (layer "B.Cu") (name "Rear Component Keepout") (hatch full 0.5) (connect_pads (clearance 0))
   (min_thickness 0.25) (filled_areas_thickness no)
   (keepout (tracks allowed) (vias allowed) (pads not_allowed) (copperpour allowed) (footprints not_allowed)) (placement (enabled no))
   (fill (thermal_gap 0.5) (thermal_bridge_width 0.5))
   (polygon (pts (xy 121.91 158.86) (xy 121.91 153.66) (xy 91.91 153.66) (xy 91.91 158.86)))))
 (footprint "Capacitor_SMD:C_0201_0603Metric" (layer "F.Cu") (at 106.26 154.09 90)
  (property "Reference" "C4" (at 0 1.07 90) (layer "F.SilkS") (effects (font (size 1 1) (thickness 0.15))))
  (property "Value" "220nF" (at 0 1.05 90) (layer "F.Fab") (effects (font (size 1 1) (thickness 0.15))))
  (pad "" smd roundrect (at -0.345 0 90) (size 0.318 0.36) (layers "F.Paste") (roundrect_rratio 0.25))
  (pad "" smd roundrect (at 0.345 0 90) (size 0.318 0.36) (layers "F.Paste") (roundrect_rratio 0.25))
  (pad "1" smd roundrect (at -0.32 0 90) (size 0.46 0.4) (layers "F.Cu" "F.Mask") (roundrect_rratio 0.25) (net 24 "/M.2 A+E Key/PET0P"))
  (pad "2" smd roundrect (at 0.32 0 90) (size 0.46 0.4) (layers "F.Cu" "F.Mask") (roundrect_rratio 0.25) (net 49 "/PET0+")))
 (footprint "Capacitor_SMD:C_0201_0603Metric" (layer "F.Cu") (at 99.56 154.09 90)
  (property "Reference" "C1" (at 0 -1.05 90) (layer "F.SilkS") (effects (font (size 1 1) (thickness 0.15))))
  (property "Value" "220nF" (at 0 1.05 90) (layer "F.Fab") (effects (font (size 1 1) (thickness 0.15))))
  (pad "" smd roundrect (at -0.345 0 90) (size 0.318 0.36) (layers "F.Paste") (roundrect_rratio 0.25))
  (pad "" smd roundrect (at 0.345 0 90) (size 0.318 0.36) (layers "F.Paste") (roundrect_rratio 0.25))
  (pad "1" smd roundrect (at -0.32 0 90) (size 0.46 0.4) (layers "F.Cu" "F.Mask") (roundrect_rratio 0.25) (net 44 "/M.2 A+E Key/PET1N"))
  (pad "2" smd roundrect (at 0.32 0 90) (size 0.46 0.4) (layers "F.Cu" "F.Mask") (roundrect_rratio 0.25) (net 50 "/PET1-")))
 (gr_line (start 117.91 154.86) (end 117.91 48.86) (stroke (width 0.1) (type default)) (layer "Edge.Cuts"))
 (gr_line (start 117.91 48.86) (end 95.91 48.86) (stroke (width 0.1) (type default)) (layer "Edge.Cuts"))
 (gr_line (start 95.91 48.86) (end 95.91 154.86) (stroke (width 0.1) (type default)) (layer "Edge.Cuts"))
 (via (at 111.91 155.09) (size 0.6) (drill 0.3) (layers "F.Cu" "B.Cu") (free yes) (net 3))
 (segment (start 111.91 155.09) (end 111.91 157.46) (width 0.2) (layer "B.Cu") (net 3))
 (segment (start 100.26 154.755001) (end 100.26 154.41) (width 0.2) (layer "F.Cu") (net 4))
 (segment (start 100.16 157.71) (end 100.16 156.434999) (width 0.2) (layer "F.Cu") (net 4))
 (segment (start 100.135 156.409999) (end 100.135 154.880001) (width 0.2) (layer "F.Cu") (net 4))
 (segment (start 100.16 156.434999) (end 100.135 156.409999) (width 0.2) (layer "F.Cu") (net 4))
 (segment (start 100.135 154.880001) (end 100.26 154.755001) (width 0.2) (layer "F.Cu") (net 4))
 (segment (start 105.685 154.880001) (end 105.56 154.755001) (width 0.2) (layer "F.Cu") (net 1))
 (segment (start 105.66 156.434999) (end 105.685 156.409999) (width 0.2) (layer "F.Cu") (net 1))
 (segment (start 105.66 157.71) (end 105.66 156.434999) (width 0.2) (layer "F.Cu") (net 1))
 (segment (start 105.56 154.755001) (end 105.56 154.41) (width 0.2) (layer "F.Cu") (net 1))
 (segment (start 105.685 156.409999) (end 105.685 154.880001) (width 0.2) (layer "F.Cu") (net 1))
 (segment (start 99.685 154.880001) (end 99.56 154.755001) (width 0.2) (layer "F.Cu") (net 44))
 (segment (start 99.66 156.434999) (end 99.685 156.409999) (width 0.2) (layer "F.Cu") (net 44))
 (segment (start 99.685 156.409999) (end 99.685 154.880001) (width 0.2) (layer "F.Cu") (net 44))
 (segment (start 99.66 157.71) (end 99.66 156.434999) (width 0.2) (layer "F.Cu") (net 44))
 (segment (start 99.56 154.755001) (end 99.56 154.41) (width 0.2) (layer "F.Cu") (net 44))
 (segment (start 106.16 156.434999) (end 106.135 156.409999) (width 0.2) (layer "F.Cu") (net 24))
 (segment (start 106.26 154.755001) (end 106.26 154.41) (width 0.2) (layer "F.Cu") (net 24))
 (segment (start 106.135 154.880001) (end 106.26 154.755001) (width 0.2) (layer "F.Cu") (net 24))
 (segment (start 106.16 157.71) (end 106.16 156.434999) (width 0.2) (layer "F.Cu") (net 24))
 (segment (start 106.135 156.409999) (end 106.135 154.880001) (width 0.2) (layer "F.Cu") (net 24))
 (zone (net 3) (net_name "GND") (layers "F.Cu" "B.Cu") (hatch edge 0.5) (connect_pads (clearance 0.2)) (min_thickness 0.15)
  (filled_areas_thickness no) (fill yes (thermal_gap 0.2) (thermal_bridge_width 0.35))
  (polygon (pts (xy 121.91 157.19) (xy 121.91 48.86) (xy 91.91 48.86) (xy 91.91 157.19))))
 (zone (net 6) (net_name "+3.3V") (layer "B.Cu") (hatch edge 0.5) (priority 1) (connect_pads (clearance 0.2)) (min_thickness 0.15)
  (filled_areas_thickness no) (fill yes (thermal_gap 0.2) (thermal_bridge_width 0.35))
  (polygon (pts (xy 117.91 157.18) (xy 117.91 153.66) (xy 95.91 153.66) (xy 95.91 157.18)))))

